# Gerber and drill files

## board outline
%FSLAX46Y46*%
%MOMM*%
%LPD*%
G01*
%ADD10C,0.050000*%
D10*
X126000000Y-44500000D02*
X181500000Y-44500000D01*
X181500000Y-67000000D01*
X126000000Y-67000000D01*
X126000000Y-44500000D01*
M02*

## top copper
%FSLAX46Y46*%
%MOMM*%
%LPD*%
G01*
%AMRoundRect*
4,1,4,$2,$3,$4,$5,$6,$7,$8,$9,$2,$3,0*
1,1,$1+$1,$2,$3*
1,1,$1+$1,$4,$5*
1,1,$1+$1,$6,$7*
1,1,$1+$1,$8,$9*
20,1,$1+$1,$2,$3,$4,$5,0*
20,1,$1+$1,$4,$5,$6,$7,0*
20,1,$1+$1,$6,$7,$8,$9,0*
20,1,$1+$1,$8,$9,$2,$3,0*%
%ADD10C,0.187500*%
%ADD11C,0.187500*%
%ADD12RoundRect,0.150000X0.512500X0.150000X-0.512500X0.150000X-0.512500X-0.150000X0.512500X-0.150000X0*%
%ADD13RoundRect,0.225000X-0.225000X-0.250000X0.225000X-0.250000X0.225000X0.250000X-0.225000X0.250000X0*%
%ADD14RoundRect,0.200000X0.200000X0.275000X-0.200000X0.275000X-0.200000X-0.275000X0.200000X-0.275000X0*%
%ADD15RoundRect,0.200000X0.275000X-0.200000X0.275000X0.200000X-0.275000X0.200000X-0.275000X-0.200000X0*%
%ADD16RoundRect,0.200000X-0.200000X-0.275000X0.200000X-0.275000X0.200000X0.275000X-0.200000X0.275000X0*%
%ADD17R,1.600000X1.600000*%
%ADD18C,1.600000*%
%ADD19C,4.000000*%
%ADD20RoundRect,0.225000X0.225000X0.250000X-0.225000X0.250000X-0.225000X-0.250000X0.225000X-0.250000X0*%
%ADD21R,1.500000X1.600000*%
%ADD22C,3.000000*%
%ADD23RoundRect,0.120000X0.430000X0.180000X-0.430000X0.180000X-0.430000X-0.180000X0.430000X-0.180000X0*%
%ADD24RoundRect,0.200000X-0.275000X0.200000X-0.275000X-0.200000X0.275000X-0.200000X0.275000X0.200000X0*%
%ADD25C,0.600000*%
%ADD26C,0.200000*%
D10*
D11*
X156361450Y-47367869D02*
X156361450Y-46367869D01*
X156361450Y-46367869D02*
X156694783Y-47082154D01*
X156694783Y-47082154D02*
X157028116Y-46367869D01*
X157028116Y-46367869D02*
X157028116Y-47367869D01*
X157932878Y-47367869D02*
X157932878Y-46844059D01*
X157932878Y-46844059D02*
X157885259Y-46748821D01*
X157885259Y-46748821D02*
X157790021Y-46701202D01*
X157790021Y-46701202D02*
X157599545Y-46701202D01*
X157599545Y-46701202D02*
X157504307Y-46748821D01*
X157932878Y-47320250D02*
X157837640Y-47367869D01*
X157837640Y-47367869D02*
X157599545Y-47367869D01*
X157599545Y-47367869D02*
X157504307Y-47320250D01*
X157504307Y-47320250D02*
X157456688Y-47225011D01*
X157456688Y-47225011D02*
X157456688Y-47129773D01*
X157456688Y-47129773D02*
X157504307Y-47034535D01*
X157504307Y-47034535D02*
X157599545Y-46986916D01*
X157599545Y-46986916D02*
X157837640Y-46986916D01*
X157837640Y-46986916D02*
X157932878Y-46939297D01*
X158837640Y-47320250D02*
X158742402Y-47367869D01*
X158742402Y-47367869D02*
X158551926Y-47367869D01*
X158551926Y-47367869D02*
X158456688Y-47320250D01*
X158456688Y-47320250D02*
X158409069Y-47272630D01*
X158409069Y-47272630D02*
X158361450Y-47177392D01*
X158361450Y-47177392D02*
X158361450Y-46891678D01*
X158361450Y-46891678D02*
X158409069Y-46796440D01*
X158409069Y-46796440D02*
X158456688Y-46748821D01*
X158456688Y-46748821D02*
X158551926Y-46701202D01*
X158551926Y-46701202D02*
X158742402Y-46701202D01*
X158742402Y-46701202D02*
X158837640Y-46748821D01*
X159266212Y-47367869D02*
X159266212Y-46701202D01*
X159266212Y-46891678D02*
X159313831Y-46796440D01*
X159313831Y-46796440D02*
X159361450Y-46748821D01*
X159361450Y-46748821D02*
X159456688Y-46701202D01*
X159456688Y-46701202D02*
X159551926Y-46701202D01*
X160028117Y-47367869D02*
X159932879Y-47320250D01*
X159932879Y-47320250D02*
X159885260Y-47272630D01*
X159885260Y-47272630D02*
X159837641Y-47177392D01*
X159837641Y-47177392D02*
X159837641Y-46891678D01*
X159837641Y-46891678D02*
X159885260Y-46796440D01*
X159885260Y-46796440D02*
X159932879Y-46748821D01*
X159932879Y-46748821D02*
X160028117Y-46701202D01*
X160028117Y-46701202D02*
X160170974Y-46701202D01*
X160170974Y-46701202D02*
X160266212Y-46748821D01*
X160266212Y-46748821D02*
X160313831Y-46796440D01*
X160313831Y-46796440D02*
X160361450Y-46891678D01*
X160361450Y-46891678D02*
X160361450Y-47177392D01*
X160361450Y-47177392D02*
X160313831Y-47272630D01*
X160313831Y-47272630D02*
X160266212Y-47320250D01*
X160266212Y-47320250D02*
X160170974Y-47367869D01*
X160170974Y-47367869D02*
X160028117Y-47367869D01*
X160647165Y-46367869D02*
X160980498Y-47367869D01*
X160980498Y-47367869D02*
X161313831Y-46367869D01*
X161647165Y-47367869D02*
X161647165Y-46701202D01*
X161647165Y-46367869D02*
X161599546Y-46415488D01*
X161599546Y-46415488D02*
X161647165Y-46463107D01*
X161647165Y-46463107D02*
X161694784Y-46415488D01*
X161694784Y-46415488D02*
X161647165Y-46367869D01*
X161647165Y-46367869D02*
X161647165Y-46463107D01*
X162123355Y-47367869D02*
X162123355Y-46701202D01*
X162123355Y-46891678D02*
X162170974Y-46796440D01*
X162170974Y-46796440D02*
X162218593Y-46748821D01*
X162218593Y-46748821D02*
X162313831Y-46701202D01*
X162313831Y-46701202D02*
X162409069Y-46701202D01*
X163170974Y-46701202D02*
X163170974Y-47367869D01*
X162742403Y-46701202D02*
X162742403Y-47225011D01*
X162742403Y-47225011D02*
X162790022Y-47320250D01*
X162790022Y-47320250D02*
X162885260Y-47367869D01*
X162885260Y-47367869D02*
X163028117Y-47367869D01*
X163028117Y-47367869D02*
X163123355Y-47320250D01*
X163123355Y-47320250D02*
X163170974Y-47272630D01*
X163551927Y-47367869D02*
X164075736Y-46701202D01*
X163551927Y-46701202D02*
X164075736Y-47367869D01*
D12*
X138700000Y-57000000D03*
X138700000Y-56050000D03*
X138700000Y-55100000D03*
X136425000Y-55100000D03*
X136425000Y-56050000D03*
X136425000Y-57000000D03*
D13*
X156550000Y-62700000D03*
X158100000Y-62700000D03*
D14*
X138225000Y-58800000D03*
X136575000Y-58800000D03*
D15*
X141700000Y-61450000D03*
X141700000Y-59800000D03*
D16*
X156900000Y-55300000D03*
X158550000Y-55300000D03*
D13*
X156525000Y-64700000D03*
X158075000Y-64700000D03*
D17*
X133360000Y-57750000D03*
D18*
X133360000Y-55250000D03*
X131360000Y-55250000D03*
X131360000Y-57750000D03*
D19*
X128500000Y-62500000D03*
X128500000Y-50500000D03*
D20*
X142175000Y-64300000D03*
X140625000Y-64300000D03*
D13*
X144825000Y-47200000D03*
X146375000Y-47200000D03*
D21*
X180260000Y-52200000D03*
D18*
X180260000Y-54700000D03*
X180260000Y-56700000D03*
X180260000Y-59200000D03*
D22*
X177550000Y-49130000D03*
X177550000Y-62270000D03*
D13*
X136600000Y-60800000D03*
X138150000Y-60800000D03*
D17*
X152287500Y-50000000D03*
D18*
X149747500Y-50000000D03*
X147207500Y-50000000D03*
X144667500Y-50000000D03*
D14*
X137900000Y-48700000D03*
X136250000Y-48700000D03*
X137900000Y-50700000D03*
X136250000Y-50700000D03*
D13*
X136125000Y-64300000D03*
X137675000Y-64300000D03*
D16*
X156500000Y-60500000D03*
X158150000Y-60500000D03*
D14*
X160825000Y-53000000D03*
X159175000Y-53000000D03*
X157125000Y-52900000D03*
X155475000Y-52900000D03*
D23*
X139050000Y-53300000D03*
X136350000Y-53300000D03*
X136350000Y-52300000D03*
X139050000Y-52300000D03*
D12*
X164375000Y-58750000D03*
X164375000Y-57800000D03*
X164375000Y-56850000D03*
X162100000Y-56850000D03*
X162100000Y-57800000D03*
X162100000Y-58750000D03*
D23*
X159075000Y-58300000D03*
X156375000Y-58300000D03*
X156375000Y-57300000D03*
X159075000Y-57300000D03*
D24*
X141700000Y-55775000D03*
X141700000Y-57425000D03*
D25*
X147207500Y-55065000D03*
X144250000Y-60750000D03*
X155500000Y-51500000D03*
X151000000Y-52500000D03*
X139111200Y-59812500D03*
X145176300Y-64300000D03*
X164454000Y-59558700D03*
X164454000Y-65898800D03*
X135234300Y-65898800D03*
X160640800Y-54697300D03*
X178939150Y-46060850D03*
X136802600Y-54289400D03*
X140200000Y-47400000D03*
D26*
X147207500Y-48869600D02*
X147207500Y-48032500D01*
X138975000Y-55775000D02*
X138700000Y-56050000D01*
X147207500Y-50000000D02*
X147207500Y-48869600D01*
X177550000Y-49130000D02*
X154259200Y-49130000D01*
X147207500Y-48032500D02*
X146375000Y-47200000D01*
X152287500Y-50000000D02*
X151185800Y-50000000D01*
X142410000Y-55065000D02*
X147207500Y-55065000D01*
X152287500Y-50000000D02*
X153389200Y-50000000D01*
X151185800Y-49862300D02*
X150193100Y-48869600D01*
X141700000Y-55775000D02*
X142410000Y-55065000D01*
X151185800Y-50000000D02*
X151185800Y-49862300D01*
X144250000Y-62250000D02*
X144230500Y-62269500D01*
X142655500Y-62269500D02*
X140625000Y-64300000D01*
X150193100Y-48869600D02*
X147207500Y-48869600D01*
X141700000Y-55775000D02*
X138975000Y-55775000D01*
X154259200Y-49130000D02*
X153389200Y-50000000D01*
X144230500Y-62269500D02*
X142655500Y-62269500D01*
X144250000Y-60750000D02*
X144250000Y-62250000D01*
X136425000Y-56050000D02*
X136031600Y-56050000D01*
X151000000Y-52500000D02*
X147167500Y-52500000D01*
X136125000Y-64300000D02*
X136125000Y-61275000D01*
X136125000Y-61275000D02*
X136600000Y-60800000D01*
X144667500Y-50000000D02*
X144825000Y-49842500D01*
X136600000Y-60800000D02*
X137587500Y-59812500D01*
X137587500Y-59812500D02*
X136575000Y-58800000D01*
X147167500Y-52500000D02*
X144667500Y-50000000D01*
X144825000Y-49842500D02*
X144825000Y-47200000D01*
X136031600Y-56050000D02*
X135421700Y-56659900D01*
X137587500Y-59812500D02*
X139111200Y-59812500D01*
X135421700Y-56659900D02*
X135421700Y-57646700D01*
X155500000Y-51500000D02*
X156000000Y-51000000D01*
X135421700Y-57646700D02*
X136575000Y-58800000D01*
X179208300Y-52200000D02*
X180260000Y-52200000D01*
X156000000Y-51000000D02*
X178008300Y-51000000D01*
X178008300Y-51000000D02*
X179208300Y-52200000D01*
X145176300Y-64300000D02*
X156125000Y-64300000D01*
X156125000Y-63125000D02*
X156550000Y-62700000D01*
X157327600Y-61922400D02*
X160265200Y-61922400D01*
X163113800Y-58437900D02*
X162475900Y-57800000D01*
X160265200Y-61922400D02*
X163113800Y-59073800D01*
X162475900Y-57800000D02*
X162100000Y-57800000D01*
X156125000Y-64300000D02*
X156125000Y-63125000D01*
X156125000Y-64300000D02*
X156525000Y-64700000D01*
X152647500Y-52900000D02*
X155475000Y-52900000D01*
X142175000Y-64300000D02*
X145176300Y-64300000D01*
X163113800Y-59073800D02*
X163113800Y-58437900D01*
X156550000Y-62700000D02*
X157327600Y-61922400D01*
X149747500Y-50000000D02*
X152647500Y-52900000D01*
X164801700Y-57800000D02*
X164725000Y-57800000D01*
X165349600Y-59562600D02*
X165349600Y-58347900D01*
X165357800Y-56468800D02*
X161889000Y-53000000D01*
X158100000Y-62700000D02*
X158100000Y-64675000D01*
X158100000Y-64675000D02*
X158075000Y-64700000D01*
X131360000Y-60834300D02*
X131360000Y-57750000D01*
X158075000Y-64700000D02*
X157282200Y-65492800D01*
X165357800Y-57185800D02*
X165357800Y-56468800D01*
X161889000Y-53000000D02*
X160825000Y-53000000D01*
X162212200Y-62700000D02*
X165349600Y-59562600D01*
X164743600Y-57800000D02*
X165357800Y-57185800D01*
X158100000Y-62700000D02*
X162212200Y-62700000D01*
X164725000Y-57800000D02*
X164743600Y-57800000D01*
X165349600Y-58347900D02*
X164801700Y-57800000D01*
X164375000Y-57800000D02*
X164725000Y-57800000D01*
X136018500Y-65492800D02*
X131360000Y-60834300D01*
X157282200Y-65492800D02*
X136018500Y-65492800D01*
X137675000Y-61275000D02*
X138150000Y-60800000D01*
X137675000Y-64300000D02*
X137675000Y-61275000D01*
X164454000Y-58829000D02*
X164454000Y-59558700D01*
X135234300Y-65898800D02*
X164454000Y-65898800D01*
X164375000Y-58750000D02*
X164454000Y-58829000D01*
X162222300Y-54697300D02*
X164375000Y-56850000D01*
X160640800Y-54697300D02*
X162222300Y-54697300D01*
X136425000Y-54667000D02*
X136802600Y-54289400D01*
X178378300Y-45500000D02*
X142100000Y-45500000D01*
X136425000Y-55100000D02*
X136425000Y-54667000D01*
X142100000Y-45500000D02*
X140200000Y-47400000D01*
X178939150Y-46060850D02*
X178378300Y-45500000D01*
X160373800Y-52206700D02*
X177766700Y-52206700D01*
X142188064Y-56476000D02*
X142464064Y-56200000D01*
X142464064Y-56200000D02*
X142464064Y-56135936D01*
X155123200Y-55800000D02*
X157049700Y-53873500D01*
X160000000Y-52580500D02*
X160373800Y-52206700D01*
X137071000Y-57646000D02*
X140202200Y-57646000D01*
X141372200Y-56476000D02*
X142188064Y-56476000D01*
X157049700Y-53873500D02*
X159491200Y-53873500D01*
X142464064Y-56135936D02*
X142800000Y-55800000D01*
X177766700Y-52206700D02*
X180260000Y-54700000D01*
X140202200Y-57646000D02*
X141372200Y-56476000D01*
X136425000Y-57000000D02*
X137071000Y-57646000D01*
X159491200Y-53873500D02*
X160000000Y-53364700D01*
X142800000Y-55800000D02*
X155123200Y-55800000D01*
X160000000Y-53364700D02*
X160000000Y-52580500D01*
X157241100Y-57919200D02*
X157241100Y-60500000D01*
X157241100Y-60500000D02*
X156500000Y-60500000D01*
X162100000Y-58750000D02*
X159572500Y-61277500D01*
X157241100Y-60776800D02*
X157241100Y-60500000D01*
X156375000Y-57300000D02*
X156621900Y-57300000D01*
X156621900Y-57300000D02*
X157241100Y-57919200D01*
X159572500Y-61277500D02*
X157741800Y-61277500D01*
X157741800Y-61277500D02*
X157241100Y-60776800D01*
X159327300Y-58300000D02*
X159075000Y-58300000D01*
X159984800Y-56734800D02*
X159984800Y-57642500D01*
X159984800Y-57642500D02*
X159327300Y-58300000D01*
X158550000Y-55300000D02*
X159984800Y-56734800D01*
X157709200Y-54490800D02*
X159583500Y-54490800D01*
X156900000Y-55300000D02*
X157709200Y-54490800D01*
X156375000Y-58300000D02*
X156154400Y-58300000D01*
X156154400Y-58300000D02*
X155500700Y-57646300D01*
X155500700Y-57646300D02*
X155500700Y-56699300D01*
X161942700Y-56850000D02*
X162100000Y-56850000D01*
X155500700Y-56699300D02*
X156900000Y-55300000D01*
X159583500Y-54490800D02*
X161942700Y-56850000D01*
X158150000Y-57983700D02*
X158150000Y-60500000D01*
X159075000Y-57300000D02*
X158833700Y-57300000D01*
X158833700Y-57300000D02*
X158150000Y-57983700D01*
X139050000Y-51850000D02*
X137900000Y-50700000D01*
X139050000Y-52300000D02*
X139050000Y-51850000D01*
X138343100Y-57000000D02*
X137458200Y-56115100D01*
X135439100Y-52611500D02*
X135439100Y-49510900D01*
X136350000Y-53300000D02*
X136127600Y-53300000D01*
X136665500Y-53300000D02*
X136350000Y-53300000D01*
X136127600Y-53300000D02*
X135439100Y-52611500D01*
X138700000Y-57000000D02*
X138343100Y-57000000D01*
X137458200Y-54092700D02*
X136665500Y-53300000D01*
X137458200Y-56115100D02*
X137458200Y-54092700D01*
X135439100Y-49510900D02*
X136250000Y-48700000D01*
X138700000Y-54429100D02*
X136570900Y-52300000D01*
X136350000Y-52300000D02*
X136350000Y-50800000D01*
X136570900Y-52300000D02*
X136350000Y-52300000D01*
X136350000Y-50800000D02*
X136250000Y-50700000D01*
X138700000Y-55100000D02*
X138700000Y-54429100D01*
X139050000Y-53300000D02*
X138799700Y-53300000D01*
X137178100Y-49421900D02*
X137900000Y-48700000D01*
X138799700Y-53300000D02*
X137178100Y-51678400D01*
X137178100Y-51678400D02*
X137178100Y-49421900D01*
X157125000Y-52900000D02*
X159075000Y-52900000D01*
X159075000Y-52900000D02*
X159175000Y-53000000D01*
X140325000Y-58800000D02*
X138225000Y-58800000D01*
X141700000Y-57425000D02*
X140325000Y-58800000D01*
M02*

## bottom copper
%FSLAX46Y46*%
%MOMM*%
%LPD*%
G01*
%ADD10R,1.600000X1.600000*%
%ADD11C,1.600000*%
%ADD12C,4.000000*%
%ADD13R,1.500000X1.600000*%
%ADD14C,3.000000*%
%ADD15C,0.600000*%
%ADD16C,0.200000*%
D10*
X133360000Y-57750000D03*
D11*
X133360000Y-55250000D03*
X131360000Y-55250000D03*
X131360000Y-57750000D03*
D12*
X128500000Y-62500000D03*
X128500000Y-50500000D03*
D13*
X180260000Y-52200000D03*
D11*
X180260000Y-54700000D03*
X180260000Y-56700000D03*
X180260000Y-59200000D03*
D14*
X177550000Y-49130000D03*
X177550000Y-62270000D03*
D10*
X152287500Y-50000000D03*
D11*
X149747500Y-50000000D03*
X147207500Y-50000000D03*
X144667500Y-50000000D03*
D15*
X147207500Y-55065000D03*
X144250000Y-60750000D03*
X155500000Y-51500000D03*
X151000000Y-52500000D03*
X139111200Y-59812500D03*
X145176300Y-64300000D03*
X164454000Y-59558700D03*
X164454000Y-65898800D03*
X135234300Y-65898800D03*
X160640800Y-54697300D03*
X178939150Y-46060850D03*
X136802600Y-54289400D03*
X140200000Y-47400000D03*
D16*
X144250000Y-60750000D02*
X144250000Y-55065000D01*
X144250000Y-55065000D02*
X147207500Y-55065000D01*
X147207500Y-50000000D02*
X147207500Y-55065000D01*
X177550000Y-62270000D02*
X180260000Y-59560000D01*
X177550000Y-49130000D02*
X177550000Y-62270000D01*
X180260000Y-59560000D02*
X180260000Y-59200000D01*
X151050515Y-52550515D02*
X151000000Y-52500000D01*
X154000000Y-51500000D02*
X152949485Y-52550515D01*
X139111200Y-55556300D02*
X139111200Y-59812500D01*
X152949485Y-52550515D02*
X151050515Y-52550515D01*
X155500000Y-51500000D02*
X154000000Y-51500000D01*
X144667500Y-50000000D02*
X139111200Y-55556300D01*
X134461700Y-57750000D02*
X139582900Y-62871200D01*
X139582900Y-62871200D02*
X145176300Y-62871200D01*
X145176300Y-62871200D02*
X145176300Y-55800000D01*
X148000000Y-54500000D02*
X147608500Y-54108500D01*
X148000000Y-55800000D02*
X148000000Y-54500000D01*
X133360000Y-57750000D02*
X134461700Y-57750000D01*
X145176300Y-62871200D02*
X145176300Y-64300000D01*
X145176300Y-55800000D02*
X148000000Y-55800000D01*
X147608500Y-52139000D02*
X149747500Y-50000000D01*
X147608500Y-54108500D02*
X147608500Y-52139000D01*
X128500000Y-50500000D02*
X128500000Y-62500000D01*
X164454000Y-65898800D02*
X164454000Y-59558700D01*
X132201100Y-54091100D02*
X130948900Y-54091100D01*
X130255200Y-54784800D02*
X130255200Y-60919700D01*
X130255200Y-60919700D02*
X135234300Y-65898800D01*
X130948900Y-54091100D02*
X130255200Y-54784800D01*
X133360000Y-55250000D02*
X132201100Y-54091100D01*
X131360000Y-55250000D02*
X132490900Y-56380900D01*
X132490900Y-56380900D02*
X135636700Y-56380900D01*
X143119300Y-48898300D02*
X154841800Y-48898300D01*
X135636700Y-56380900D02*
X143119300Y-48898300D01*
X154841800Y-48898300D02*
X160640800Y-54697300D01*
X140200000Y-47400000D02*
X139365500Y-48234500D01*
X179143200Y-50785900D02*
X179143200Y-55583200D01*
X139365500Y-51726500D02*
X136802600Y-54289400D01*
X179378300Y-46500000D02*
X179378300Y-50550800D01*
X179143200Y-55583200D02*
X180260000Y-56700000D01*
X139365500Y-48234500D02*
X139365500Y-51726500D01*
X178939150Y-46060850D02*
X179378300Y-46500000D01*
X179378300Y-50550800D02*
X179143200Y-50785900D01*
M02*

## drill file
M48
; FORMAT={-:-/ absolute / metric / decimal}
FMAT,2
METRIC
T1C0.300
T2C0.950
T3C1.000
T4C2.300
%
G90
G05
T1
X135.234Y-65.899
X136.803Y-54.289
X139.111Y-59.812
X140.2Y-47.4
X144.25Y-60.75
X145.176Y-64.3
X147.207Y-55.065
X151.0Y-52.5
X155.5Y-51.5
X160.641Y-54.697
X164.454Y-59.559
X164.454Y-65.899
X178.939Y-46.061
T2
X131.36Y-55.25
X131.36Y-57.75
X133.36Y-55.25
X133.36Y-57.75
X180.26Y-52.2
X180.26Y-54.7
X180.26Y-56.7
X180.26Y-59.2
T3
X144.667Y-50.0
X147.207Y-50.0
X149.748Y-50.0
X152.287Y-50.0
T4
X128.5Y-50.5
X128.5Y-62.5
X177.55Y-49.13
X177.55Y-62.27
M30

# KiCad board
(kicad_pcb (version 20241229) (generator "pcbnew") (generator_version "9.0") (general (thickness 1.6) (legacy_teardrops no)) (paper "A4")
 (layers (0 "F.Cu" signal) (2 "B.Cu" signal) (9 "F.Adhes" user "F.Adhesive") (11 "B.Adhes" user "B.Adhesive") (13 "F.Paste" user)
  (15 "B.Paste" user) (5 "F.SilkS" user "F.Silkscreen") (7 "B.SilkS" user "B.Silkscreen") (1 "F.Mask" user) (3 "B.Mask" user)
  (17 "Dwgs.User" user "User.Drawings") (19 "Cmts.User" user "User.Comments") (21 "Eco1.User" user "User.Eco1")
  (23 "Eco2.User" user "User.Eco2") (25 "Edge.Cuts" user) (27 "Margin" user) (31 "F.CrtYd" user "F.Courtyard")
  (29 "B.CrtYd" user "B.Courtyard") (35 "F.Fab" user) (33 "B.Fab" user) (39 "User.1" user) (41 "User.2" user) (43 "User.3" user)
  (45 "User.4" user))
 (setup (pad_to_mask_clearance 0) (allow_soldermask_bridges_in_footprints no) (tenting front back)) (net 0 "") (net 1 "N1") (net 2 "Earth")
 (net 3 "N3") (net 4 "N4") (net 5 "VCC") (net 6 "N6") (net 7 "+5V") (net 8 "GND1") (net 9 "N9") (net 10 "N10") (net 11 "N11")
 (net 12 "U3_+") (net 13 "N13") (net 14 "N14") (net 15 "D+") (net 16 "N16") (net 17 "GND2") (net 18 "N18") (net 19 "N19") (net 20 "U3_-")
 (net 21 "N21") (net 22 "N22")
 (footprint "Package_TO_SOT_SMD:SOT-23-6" (layer "F.Cu") (at 137.5625 56.05 180)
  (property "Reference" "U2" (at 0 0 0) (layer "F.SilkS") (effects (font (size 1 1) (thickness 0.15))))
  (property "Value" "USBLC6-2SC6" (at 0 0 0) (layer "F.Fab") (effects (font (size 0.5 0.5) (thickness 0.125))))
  (pad "1" smd roundrect (at -1.1375 -0.95 180) (size 1.325 0.6) (layers "F.Cu" "F.Mask" "F.Paste") (roundrect_rratio 0.25) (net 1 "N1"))
  (pad "2" smd roundrect (at -1.1375 0 180) (size 1.325 0.6) (layers "F.Cu" "F.Mask" "F.Paste") (roundrect_rratio 0.25) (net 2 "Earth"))
  (pad "3" smd roundrect (at -1.1375 0.95 180) (size 1.325 0.6) (layers "F.Cu" "F.Mask" "F.Paste") (roundrect_rratio 0.25) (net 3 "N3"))
  (pad "4" smd roundrect (at 1.1375 0.95 180) (size 1.325 0.6) (layers "F.Cu" "F.Mask" "F.Paste") (roundrect_rratio 0.25) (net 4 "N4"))
  (pad "5" smd roundrect (at 1.1375 0 180) (size 1.325 0.6) (layers "F.Cu" "F.Mask" "F.Paste") (roundrect_rratio 0.25) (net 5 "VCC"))
  (pad "6" smd roundrect (at 1.1375 -0.95 180) (size 1.325 0.6) (layers "F.Cu" "F.Mask" "F.Paste") (roundrect_rratio 0.25) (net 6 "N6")))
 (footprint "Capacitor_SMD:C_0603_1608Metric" (layer "F.Cu") (at 157.325 62.7)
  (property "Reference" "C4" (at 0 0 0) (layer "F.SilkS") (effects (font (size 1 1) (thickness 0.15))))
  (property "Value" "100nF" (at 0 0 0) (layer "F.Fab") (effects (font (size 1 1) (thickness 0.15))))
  (pad "1" smd roundrect (at -0.775 0) (size 0.9 0.95) (layers "F.Cu" "F.Mask" "F.Paste") (roundrect_rratio 0.25) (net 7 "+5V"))
  (pad "2" smd roundrect (at 0.775 0) (size 0.9 0.95) (layers "F.Cu" "F.Mask" "F.Paste") (roundrect_rratio 0.25) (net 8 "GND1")))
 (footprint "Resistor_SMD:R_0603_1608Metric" (layer "F.Cu") (at 137.4 58.8 180)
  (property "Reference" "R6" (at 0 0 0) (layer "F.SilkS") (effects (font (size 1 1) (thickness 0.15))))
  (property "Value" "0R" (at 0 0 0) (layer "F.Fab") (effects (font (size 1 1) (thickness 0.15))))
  (pad "1" smd roundrect (at -0.825 0 180) (size 0.8 0.95) (layers "F.Cu" "F.Mask" "F.Paste") (roundrect_rratio 0.25) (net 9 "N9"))
  (pad "2" smd roundrect (at 0.825 0 180) (size 0.8 0.95) (layers "F.Cu" "F.Mask" "F.Paste") (roundrect_rratio 0.25) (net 5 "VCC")))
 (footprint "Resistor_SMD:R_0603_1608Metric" (layer "F.Cu") (at 141.7 60.625 90)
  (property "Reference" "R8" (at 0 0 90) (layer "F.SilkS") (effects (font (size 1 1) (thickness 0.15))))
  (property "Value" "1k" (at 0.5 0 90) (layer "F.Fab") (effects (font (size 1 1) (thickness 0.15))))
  (pad "1" smd roundrect (at -0.825 0 90) (size 0.8 0.95) (layers "F.Cu" "F.Mask" "F.Paste") (roundrect_rratio 0.25) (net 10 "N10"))
  (pad "2" smd roundrect (at 0.825 0 90) (size 0.8 0.95) (layers "F.Cu" "F.Mask" "F.Paste") (roundrect_rratio 0.25) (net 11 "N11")))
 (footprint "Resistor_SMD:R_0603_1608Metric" (layer "F.Cu") (at 157.725 55.3)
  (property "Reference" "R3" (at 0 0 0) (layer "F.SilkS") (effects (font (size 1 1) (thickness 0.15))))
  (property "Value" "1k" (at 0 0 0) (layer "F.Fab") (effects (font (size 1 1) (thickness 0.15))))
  (pad "1" smd roundrect (at -0.825 0) (size 0.8 0.95) (layers "F.Cu" "F.Mask" "F.Paste") (roundrect_rratio 0.25) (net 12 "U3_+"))
  (pad "2" smd roundrect (at 0.825 0) (size 0.8 0.95) (layers "F.Cu" "F.Mask" "F.Paste") (roundrect_rratio 0.25) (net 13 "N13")))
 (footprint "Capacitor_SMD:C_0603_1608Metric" (layer "F.Cu") (at 157.3 64.7)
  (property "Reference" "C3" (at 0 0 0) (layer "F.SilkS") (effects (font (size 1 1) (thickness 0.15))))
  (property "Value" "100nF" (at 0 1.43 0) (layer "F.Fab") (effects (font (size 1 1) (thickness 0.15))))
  (pad "1" smd roundrect (at -0.775 0) (size 0.9 0.95) (layers "F.Cu" "F.Mask" "F.Paste") (roundrect_rratio 0.25) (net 7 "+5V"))
  (pad "2" smd roundrect (at 0.775 0) (size 0.9 0.95) (layers "F.Cu" "F.Mask" "F.Paste") (roundrect_rratio 0.25) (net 8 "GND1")))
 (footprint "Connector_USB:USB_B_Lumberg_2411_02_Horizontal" (layer "F.Cu") (at 133.36 57.75 180)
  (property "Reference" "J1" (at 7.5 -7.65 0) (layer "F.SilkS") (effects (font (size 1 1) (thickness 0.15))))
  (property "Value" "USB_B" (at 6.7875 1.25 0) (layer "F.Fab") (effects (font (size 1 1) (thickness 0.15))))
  (pad "1" thru_hole rect (at 0 0 270) (size 1.6 1.6) (drill 0.95) (layers "*.Cu" "*.Mask") (remove_unused_layers no) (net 7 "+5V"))
  (pad "2" thru_hole circle (at 0 2.5 270) (size 1.6 1.6) (drill 0.95) (layers "*.Cu" "*.Mask") (remove_unused_layers no) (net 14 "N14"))
  (pad "3" thru_hole circle (at 2 2.5 270) (size 1.6 1.6) (drill 0.95) (layers "*.Cu" "*.Mask") (remove_unused_layers no) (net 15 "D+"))
  (pad "4" thru_hole circle (at 2 0 270) (size 1.6 1.6) (drill 0.95) (layers "*.Cu" "*.Mask") (remove_unused_layers no) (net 8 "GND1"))
  (pad "5" thru_hole circle (at 4.86 -4.75 270) (size 4 4) (drill 2.3) (layers "*.Cu" "*.Mask") (remove_unused_layers no) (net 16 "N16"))
  (pad "5" thru_hole circle (at 4.86 7.25 270) (size 4 4) (drill 2.3) (layers "*.Cu" "*.Mask") (remove_unused_layers no) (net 16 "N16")))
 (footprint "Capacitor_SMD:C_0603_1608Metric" (layer "F.Cu") (at 141.4 64.3 180)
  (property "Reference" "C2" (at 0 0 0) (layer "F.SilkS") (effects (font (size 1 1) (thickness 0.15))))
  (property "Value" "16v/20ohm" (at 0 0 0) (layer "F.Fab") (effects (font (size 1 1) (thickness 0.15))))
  (pad "1" smd roundrect (at -0.775 0 180) (size 0.9 0.95) (layers "F.Cu" "F.Mask" "F.Paste") (roundrect_rratio 0.25) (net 7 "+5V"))
  (pad "2" smd roundrect (at 0.775 0 180) (size 0.9 0.95) (layers "F.Cu" "F.Mask" "F.Paste") (roundrect_rratio 0.25) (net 2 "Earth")))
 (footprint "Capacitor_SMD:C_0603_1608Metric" (layer "F.Cu") (at 145.6 47.2)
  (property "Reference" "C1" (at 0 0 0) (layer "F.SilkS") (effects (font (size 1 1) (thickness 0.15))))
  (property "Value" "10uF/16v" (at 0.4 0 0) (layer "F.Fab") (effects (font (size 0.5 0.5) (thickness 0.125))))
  (pad "1" smd roundrect (at -0.775 0) (size 0.9 0.95) (layers "F.Cu" "F.Mask" "F.Paste") (roundrect_rratio 0.25) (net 5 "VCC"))
  (pad "2" smd roundrect (at 0.775 0) (size 0.9 0.95) (layers "F.Cu" "F.Mask" "F.Paste") (roundrect_rratio 0.25) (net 2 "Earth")))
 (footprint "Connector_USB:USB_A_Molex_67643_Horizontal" (layer "F.Cu") (at 180.26 52.2 -90)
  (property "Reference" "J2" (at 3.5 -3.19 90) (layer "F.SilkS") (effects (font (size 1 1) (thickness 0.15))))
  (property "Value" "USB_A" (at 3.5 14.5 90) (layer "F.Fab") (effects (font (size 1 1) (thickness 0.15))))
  (pad "1" thru_hole rect (at 0 0 270) (size 1.6 1.5) (drill 0.95) (layers "*.Cu" "*.Mask") (remove_unused_layers no) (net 5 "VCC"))
  (pad "2" thru_hole circle (at 2.5 0 270) (size 1.6 1.6) (drill 0.95) (layers "*.Cu" "*.Mask") (remove_unused_layers no) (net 6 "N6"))
  (pad "3" thru_hole circle (at 4.5 0 270) (size 1.6 1.6) (drill 0.95) (layers "*.Cu" "*.Mask") (remove_unused_layers no) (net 4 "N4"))
  (pad "4" thru_hole circle (at 7 0 270) (size 1.6 1.6) (drill 0.95) (layers "*.Cu" "*.Mask") (remove_unused_layers no) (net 2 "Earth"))
  (pad "5" thru_hole circle (at -3.07 2.71 270) (size 3 3) (drill 2.3) (layers "*.Cu" "*.Mask") (remove_unused_layers no) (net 2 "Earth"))
  (pad "5" thru_hole circle (at 10.07 2.71 270) (size 3 3) (drill 2.3) (layers "*.Cu" "*.Mask") (remove_unused_layers no) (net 2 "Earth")))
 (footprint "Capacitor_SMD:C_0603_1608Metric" (layer "F.Cu") (at 137.375 60.8)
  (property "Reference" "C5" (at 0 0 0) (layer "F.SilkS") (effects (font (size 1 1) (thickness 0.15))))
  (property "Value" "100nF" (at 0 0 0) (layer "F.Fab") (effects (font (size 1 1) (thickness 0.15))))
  (pad "1" smd roundrect (at -0.775 0) (size 0.9 0.95) (layers "F.Cu" "F.Mask" "F.Paste") (roundrect_rratio 0.25) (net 5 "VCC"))
  (pad "2" smd roundrect (at 0.775 0) (size 0.9 0.95) (layers "F.Cu" "F.Mask" "F.Paste") (roundrect_rratio 0.25) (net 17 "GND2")))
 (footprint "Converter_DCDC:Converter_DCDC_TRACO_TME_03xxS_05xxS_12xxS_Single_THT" (layer "F.Cu") (at 152.2875 50 -90)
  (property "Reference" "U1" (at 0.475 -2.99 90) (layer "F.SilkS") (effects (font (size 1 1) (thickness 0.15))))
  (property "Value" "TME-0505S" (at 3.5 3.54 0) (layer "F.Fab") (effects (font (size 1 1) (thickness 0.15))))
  (pad "1" thru_hole rect (at 0 0 270) (size 1.6 1.6) (drill 1) (layers "*.Cu" "*.Mask") (remove_unused_layers no) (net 2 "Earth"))
  (pad "2" thru_hole circle (at 0 2.54 270) (size 1.6 1.6) (drill 1) (layers "*.Cu" "*.Mask") (remove_unused_layers no) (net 7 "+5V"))
  (pad "3" thru_hole circle (at 0 5.08 270) (size 1.6 1.6) (drill 1) (layers "*.Cu" "*.Mask") (remove_unused_layers no) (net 2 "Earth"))
  (pad "4" thru_hole circle (at 0 7.62 270) (size 1.6 1.6) (drill 1) (layers "*.Cu" "*.Mask") (remove_unused_layers no) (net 5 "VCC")))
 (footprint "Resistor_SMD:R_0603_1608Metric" (layer "F.Cu") (at 137.075 48.7 180)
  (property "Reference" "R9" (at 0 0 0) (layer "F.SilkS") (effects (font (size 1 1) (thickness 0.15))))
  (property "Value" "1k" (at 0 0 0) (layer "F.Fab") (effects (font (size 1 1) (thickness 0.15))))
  (pad "1" smd roundrect (at -0.825 0 180) (size 0.8 0.95) (layers "F.Cu" "F.Mask" "F.Paste") (roundrect_rratio 0.25) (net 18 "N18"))
  (pad "2" smd roundrect (at 0.825 0 180) (size 0.8 0.95) (layers "F.Cu" "F.Mask" "F.Paste") (roundrect_rratio 0.25) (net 1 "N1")))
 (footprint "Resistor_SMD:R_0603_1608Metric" (layer "F.Cu") (at 137.075 50.7 180)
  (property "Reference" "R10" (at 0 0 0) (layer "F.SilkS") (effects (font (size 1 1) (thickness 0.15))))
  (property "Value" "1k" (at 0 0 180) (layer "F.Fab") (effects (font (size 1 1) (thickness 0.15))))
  (pad "1" smd roundrect (at -0.825 0 180) (size 0.8 0.95) (layers "F.Cu" "F.Mask" "F.Paste") (roundrect_rratio 0.25) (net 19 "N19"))
  (pad "2" smd roundrect (at 0.825 0 180) (size 0.8 0.95) (layers "F.Cu" "F.Mask" "F.Paste") (roundrect_rratio 0.25) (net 3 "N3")))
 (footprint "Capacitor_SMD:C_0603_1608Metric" (layer "F.Cu") (at 136.9 64.3)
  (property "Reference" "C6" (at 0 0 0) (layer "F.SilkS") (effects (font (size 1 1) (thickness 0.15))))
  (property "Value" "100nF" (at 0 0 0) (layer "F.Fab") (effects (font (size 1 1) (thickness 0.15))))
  (pad "1" smd roundrect (at -0.775 0) (size 0.9 0.95) (layers "F.Cu" "F.Mask" "F.Paste") (roundrect_rratio 0.25) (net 5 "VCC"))
  (pad "2" smd roundrect (at 0.775 0) (size 0.9 0.95) (layers "F.Cu" "F.Mask" "F.Paste") (roundrect_rratio 0.25) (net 17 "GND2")))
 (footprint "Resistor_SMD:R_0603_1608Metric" (layer "F.Cu") (at 157.325 60.5)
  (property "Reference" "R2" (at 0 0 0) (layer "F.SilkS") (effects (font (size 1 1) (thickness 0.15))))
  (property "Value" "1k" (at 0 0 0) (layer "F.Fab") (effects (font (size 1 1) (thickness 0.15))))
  (pad "1" smd roundrect (at -0.825 0) (size 0.8 0.95) (layers "F.Cu" "F.Mask" "F.Paste") (roundrect_rratio 0.25) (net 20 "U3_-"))
  (pad "2" smd roundrect (at 0.825 0) (size 0.8 0.95) (layers "F.Cu" "F.Mask" "F.Paste") (roundrect_rratio 0.25) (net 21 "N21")))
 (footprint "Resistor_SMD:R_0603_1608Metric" (layer "F.Cu") (at 160 53 180)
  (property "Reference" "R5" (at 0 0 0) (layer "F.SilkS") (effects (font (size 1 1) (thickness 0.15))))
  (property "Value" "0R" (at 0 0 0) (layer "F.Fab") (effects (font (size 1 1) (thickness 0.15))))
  (pad "1" smd roundrect (at -0.825 0 180) (size 0.8 0.95) (layers "F.Cu" "F.Mask" "F.Paste") (roundrect_rratio 0.25) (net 8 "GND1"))
  (pad "2" smd roundrect (at 0.825 0 180) (size 0.8 0.95) (layers "F.Cu" "F.Mask" "F.Paste") (roundrect_rratio 0.25) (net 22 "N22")))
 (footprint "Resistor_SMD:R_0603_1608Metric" (layer "F.Cu") (at 156.3 52.9 180)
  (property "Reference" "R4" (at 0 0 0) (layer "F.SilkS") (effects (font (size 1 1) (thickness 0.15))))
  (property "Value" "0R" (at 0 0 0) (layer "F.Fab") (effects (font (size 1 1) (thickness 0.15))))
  (pad "1" smd roundrect (at -0.825 0 180) (size 0.8 0.95) (layers "F.Cu" "F.Mask" "F.Paste") (roundrect_rratio 0.25) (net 22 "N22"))
  (pad "2" smd roundrect (at 0.825 0 180) (size 0.8 0.95) (layers "F.Cu" "F.Mask" "F.Paste") (roundrect_rratio 0.25) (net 7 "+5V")))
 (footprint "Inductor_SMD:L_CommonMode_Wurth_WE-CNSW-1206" (layer "F.Cu") (at 137.7 52.8 180)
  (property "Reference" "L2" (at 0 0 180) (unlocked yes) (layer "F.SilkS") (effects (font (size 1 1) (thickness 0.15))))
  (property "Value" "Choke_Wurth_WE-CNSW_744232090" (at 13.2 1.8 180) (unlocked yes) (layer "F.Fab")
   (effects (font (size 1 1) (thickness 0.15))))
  (pad "1" smd roundrect (at -1.35 -0.5 180) (size 1.1 0.6) (layers "F.Cu" "F.Mask" "F.Paste") (roundrect_rratio 0.2) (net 18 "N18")
   (thermal_bridge_angle 45))
  (pad "2" smd roundrect (at 1.35 -0.5 180) (size 1.1 0.6) (layers "F.Cu" "F.Mask" "F.Paste") (roundrect_rratio 0.2) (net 1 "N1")
   (thermal_bridge_angle 45))
  (pad "3" smd roundrect (at 1.35 0.5 180) (size 1.1 0.6) (layers "F.Cu" "F.Mask" "F.Paste") (roundrect_rratio 0.2) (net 3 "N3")
   (thermal_bridge_angle 45))
  (pad "4" smd roundrect (at -1.35 0.5 180) (size 1.1 0.6) (layers "F.Cu" "F.Mask" "F.Paste") (roundrect_rratio 0.2) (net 19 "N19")
   (thermal_bridge_angle 45)))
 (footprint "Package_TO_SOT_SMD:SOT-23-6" (layer "F.Cu") (at 163.2375 57.8 180)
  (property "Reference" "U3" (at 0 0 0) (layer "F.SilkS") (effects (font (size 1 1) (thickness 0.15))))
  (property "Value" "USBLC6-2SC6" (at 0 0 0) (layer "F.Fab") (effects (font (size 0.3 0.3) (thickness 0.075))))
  (pad "1" smd roundrect (at -1.1375 -0.95 180) (size 1.325 0.6) (layers "F.Cu" "F.Mask" "F.Paste") (roundrect_rratio 0.25) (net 14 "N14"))
  (pad "2" smd roundrect (at -1.1375 0 180) (size 1.325 0.6) (layers "F.Cu" "F.Mask" "F.Paste") (roundrect_rratio 0.25) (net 8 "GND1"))
  (pad "3" smd roundrect (at -1.1375 0.95 180) (size 1.325 0.6) (layers "F.Cu" "F.Mask" "F.Paste") (roundrect_rratio 0.25) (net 15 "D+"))
  (pad "4" smd roundrect (at 1.1375 0.95 180) (size 1.325 0.6) (layers "F.Cu" "F.Mask" "F.Paste") (roundrect_rratio 0.25) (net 12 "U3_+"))
  (pad "5" smd roundrect (at 1.1375 0 180) (size 1.325 0.6) (layers "F.Cu" "F.Mask" "F.Paste") (roundrect_rratio 0.25) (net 7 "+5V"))
  (pad "6" smd roundrect (at 1.1375 -0.95 180) (size 1.325 0.6) (layers "F.Cu" "F.Mask" "F.Paste") (roundrect_rratio 0.25) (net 20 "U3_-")))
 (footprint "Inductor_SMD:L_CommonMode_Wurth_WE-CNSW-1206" (layer "F.Cu") (at 157.725 57.8 180)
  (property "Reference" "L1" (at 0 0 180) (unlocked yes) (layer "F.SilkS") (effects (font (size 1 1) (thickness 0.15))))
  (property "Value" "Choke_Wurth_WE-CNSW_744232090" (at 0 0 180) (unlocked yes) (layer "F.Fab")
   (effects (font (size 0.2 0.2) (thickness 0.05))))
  (pad "1" smd roundrect (at -1.35 -0.5 180) (size 1.1 0.6) (layers "F.Cu" "F.Mask" "F.Paste") (roundrect_rratio 0.2) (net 13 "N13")
   (thermal_bridge_angle 45))
  (pad "2" smd roundrect (at 1.35 -0.5 180) (size 1.1 0.6) (layers "F.Cu" "F.Mask" "F.Paste") (roundrect_rratio 0.2) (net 12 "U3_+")
   (thermal_bridge_angle 45))
  (pad "3" smd roundrect (at 1.35 0.5 180) (size 1.1 0.6) (layers "F.Cu" "F.Mask" "F.Paste") (roundrect_rratio 0.2) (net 20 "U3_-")
   (thermal_bridge_angle 45))
  (pad "4" smd roundrect (at -1.35 0.5 180) (size 1.1 0.6) (layers "F.Cu" "F.Mask" "F.Paste") (roundrect_rratio 0.2) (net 21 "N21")
   (thermal_bridge_angle 45)))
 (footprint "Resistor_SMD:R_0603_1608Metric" (layer "F.Cu") (at 141.7 56.6 -90)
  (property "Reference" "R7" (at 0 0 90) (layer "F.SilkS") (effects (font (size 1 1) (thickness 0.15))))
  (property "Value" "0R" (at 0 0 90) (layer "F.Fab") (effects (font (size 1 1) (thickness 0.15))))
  (pad "1" smd roundrect (at -0.825 0 270) (size 0.8 0.95) (layers "F.Cu" "F.Mask" "F.Paste") (roundrect_rratio 0.25) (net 2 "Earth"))
  (pad "2" smd roundrect (at 0.825 0 270) (size 0.8 0.95) (layers "F.Cu" "F.Mask" "F.Paste") (roundrect_rratio 0.25) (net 9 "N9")))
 (gr_rect (start 126 44.5) (end 181.5 67) (stroke (width 0.05) (type default)) (fill no) (layer "Edge.Cuts"))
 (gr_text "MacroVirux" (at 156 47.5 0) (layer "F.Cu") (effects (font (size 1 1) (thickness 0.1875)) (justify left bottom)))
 (segment (start 147.2075 48.8696) (end 147.2075 48.0325) (width 0.2) (layer "F.Cu") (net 2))
 (segment (start 138.975 55.775) (end 138.7 56.05) (width 0.2) (layer "F.Cu") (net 2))
 (segment (start 147.2075 50) (end 147.2075 48.8696) (width 0.2) (layer "F.Cu") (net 2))
 (segment (start 177.55 49.13) (end 154.2592 49.13) (width 0.2) (layer "F.Cu") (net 2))
 (segment (start 147.2075 48.0325) (end 146.375 47.2) (width 0.2) (layer "F.Cu") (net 2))
 (segment (start 152.2875 50) (end 151.1858 50) (width 0.2) (layer "F.Cu") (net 2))
 (segment (start 142.41 55.065) (end 147.2075 55.065) (width 0.2) (layer "F.Cu") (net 2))
 (segment (start 152.2875 50) (end 153.3892 50) (width 0.2) (layer "F.Cu") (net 2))
 (segment (start 151.1858 49.8623) (end 150.1931 48.8696) (width 0.2) (layer "F.Cu") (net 2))
 (segment (start 141.7 55.775) (end 142.41 55.065) (width 0.2) (layer "F.Cu") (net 2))
 (segment (start 151.1858 50) (end 151.1858 49.8623) (width 0.2) (layer "F.Cu") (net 2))
 (segment (start 144.25 62.25) (end 144.2305 62.2695) (width 0.2) (layer "F.Cu") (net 2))
 (segment (start 142.6555 62.2695) (end 140.625 64.3) (width 0.2) (layer "F.Cu") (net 2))
 (segment (start 150.1931 48.8696) (end 147.2075 48.8696) (width 0.2) (layer "F.Cu") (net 2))
 (segment (start 141.7 55.775) (end 138.975 55.775) (width 0.2) (layer "F.Cu") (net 2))
 (segment (start 154.2592 49.13) (end 153.3892 50) (width 0.2) (layer "F.Cu") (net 2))
 (segment (start 144.2305 62.2695) (end 142.6555 62.2695) (width 0.2) (layer "F.Cu") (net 2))
 (segment (start 144.25 60.75) (end 144.25 62.25) (width 0.2) (layer "F.Cu") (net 2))
 (via (at 147.2075 55.065) (size 0.6) (drill 0.3) (layers "F.Cu" "B.Cu") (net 2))
 (via (at 144.25 60.75) (size 0.6) (drill 0.3) (layers "F.Cu" "B.Cu") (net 2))
 (segment (start 144.25 60.75) (end 144.25 55.065) (width 0.2) (layer "B.Cu") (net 2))
 (segment (start 144.25 55.065) (end 147.2075 55.065) (width 0.2) (layer "B.Cu") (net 2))
 (segment (start 147.2075 50) (end 147.2075 55.065) (width 0.2) (layer "B.Cu") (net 2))
 (segment (start 177.55 62.27) (end 180.26 59.56) (width 0.2) (layer "B.Cu") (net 2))
 (segment (start 177.55 49.13) (end 177.55 62.27) (width 0.2) (layer "B.Cu") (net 2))
 (segment (start 180.26 59.56) (end 180.26 59.2) (width 0.2) (layer "B.Cu") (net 2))
 (segment (start 136.425 56.05) (end 136.0316 56.05) (width 0.2) (layer "F.Cu") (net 5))
 (segment (start 151 52.5) (end 147.1675 52.5) (width 0.2) (layer "F.Cu") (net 5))
 (segment (start 136.125 64.3) (end 136.125 61.275) (width 0.2) (layer "F.Cu") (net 5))
 (segment (start 136.125 61.275) (end 136.6 60.8) (width 0.2) (layer "F.Cu") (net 5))
 (segment (start 144.6675 50) (end 144.825 49.8425) (width 0.2) (layer "F.Cu") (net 5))
 (segment (start 136.6 60.8) (end 137.5875 59.8125) (width 0.2) (layer "F.Cu") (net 5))
 (segment (start 137.5875 59.8125) (end 136.575 58.8) (width 0.2) (layer "F.Cu") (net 5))
 (segment (start 147.1675 52.5) (end 144.6675 50) (width 0.2) (layer "F.Cu") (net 5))
 (segment (start 144.825 49.8425) (end 144.825 47.2) (width 0.2) (layer "F.Cu") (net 5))
 (segment (start 136.0316 56.05) (end 135.4217 56.6599) (width 0.2) (layer "F.Cu") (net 5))
 (segment (start 137.5875 59.8125) (end 139.1112 59.8125) (width 0.2) (layer "F.Cu") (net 5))
 (segment (start 135.4217 56.6599) (end 135.4217 57.6467) (width 0.2) (layer "F.Cu") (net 5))
 (segment (start 155.5 51.5) (end 156 51) (width 0.2) (layer "F.Cu") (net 5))
 (segment (start 135.4217 57.6467) (end 136.575 58.8) (width 0.2) (layer "F.Cu") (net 5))
 (segment (start 179.2083 52.2) (end 180.26 52.2) (width 0.2) (layer "F.Cu") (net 5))
 (segment (start 156 51) (end 178.0083 51) (width 0.2) (layer "F.Cu") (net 5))
 (segment (start 178.0083 51) (end 179.2083 52.2) (width 0.2) (layer "F.Cu") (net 5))
 (via (at 155.5 51.5) (size 0.6) (drill 0.3) (layers "F.Cu" "B.Cu") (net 5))
 (via (at 151 52.5) (size 0.6) (drill 0.3) (layers "F.Cu" "B.Cu") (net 5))
 (via (at 139.1112 59.8125) (size 0.6) (drill 0.3) (layers "F.Cu" "B.Cu") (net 5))
 (segment (start 151.050515 52.550515) (end 151 52.5) (width 0.2) (layer "B.Cu") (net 5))
 (segment (start 154 51.5) (end 152.949485 52.550515) (width 0.2) (layer "B.Cu") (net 5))
 (segment (start 139.1112 55.5563) (end 139.1112 59.8125) (width 0.2) (layer "B.Cu") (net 5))
 (segment (start 152.949485 52.550515) (end 151.050515 52.550515) (width 0.2) (layer "B.Cu") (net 5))
 (segment (start 155.5 51.5) (end 154 51.5) (width 0.2) (layer "B.Cu") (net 5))
 (segment (start 144.6675 50) (end 139.1112 55.5563) (width 0.2) (layer "B.Cu") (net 5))
 (segment (start 145.1763 64.3) (end 156.125 64.3) (width 0.2) (layer "F.Cu") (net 7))
 (segment (start 156.125 63.125) (end 156.55 62.7) (width 0.2) (layer "F.Cu") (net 7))
 (segment (start 157.3276 61.9224) (end 160.2652 61.9224) (width 0.2) (layer "F.Cu") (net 7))
 (segment (start 163.1138 58.4379) (end 162.4759 57.8) (width 0.2) (layer "F.Cu") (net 7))
 (segment (start 160.2652 61.9224) (end 163.1138 59.0738) (width 0.2) (layer "F.Cu") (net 7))
 (segment (start 162.4759 57.8) (end 162.1 57.8) (width 0.2) (layer "F.Cu") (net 7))
 (segment (start 156.125 64.3) (end 156.125 63.125) (width 0.2) (layer "F.Cu") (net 7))
 (segment (start 156.125 64.3) (end 156.525 64.7) (width 0.2) (layer "F.Cu") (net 7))
 (segment (start 152.6475 52.9) (end 155.475 52.9) (width 0.2) (layer "F.Cu") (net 7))
 (segment (start 142.175 64.3) (end 145.1763 64.3) (width 0.2) (layer "F.Cu") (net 7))
 (segment (start 163.1138 59.0738) (end 163.1138 58.4379) (width 0.2) (layer "F.Cu") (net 7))
 (segment (start 156.55 62.7) (end 157.3276 61.9224) (width 0.2) (layer "F.Cu") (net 7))
 (segment (start 149.7475 50) (end 152.6475 52.9) (width 0.2) (layer "F.Cu") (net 7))
 (via (at 145.1763 64.3) (size 0.6) (drill 0.3) (layers "F.Cu" "B.Cu") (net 7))
 (segment (start 134.4617 57.75) (end 139.5829 62.8712) (width 0.2) (layer "B.Cu") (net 7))
 (segment (start 139.5829 62.8712) (end 145.1763 62.8712) (width 0.2) (layer "B.Cu") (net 7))
 (segment (start 145.1763 62.8712) (end 145.1763 55.8) (width 0.2) (layer "B.Cu") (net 7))
 (segment (start 148 54.5) (end 147.6085 54.1085) (width 0.2) (layer "B.Cu") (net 7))
 (segment (start 148 55.8) (end 148 54.5) (width 0.2) (layer "B.Cu") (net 7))
 (segment (start 133.36 57.75) (end 134.4617 57.75) (width 0.2) (layer "B.Cu") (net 7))
 (segment (start 145.1763 62.8712) (end 145.1763 64.3) (width 0.2) (layer "B.Cu") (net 7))
 (segment (start 145.1763 55.8) (end 148 55.8) (width 0.2) (layer "B.Cu") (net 7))
 (segment (start 147.6085 52.139) (end 149.7475 50) (width 0.2) (layer "B.Cu") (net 7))
 (segment (start 147.6085 54.1085) (end 147.6085 52.139) (width 0.2) (layer "B.Cu") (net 7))
 (segment (start 164.8017 57.8) (end 164.725 57.8) (width 0.2) (layer "F.Cu") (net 8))
 (segment (start 165.3496 59.5626) (end 165.3496 58.3479) (width 0.2) (layer "F.Cu") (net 8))
 (segment (start 165.3578 56.4688) (end 161.889 53) (width 0.2) (layer "F.Cu") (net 8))
 (segment (start 158.1 62.7) (end 158.1 64.675) (width 0.2) (layer "F.Cu") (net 8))
 (segment (start 158.1 64.675) (end 158.075 64.7) (width 0.2) (layer "F.Cu") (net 8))
 (segment (start 131.36 60.8343) (end 131.36 57.75) (width 0.2) (layer "F.Cu") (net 8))
 (segment (start 158.075 64.7) (end 157.2822 65.4928) (width 0.2) (layer "F.Cu") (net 8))
 (segment (start 165.3578 57.1858) (end 165.3578 56.4688) (width 0.2) (layer "F.Cu") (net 8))
 (segment (start 161.889 53) (end 160.825 53) (width 0.2) (layer "F.Cu") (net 8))
 (segment (start 162.2122 62.7) (end 165.3496 59.5626) (width 0.2) (layer "F.Cu") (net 8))
 (segment (start 164.7436 57.8) (end 165.3578 57.1858) (width 0.2) (layer "F.Cu") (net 8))
 (segment (start 158.1 62.7) (end 162.2122 62.7) (width 0.2) (layer "F.Cu") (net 8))
 (segment (start 164.725 57.8) (end 164.7436 57.8) (width 0.2) (layer "F.Cu") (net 8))
 (segment (start 165.3496 58.3479) (end 164.8017 57.8) (width 0.2) (layer "F.Cu") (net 8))
 (segment (start 164.375 57.8) (end 164.725 57.8) (width 0.2) (layer "F.Cu") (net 8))
 (segment (start 136.0185 65.4928) (end 131.36 60.8343) (width 0.2) (layer "F.Cu") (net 8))
 (segment (start 157.2822 65.4928) (end 136.0185 65.4928) (width 0.2) (layer "F.Cu") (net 8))
 (segment (start 137.675 61.275) (end 138.15 60.8) (width 0.2) (layer "F.Cu") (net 17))
 (segment (start 137.675 64.3) (end 137.675 61.275) (width 0.2) (layer "F.Cu") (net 17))
 (segment (start 128.5 50.5) (end 128.5 62.5) (width 0.2) (layer "B.Cu") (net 16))
 (segment (start 164.454 58.829) (end 164.454 59.5587) (width 0.2) (layer "F.Cu") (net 14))
 (segment (start 135.2343 65.8988) (end 164.454 65.8988) (width 0.2) (layer "F.Cu") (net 14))
 (segment (start 164.375 58.75) (end 164.454 58.829) (width 0.2) (layer "F.Cu") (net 14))
 (via (at 164.454 59.5587) (size 0.6) (drill 0.3) (layers "F.Cu" "B.Cu") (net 14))
 (via (at 164.454 65.8988) (size 0.6) (drill 0.3) (layers "F.Cu" "B.Cu") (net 14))
 (via (at 135.2343 65.8988) (size 0.6) (drill 0.3) (layers "F.Cu" "B.Cu") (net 14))
 (segment (start 164.454 65.8988) (end 164.454 59.5587) (width 0.2) (layer "B.Cu") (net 14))
 (segment (start 132.2011 54.0911) (end 130.9489 54.0911) (width 0.2) (layer "B.Cu") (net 14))
 (segment (start 130.2552 54.7848) (end 130.2552 60.9197) (width 0.2) (layer "B.Cu") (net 14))
 (segment (start 130.2552 60.9197) (end 135.2343 65.8988) (width 0.2) (layer "B.Cu") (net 14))
 (segment (start 130.9489 54.0911) (end 130.2552 54.7848) (width 0.2) (layer "B.Cu") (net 14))
 (segment (start 133.36 55.25) (end 132.2011 54.0911) (width 0.2) (layer "B.Cu") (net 14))
 (segment (start 162.2223 54.6973) (end 164.375 56.85) (width 0.2) (layer "F.Cu") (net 15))
 (segment (start 160.6408 54.6973) (end 162.2223 54.6973) (width 0.2) (layer "F.Cu") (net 15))
 (via (at 160.6408 54.6973) (size 0.6) (drill 0.3) (layers "F.Cu" "B.Cu") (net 15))
 (segment (start 131.36 55.25) (end 132.4909 56.3809) (width 0.2) (layer "B.Cu") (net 15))
 (segment (start 132.4909 56.3809) (end 135.6367 56.3809) (width 0.2) (layer "B.Cu") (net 15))
 (segment (start 143.1193 48.8983) (end 154.8418 48.8983) (width 0.2) (layer "B.Cu") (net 15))
 (segment (start 135.6367 56.3809) (end 143.1193 48.8983) (width 0.2) (layer "B.Cu") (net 15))
 (segment (start 154.8418 48.8983) (end 160.6408 54.6973) (width 0.2) (layer "B.Cu") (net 15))
 (segment (start 136.425 54.667) (end 136.8026 54.2894) (width 0.2) (layer "F.Cu") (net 4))
 (segment (start 178.3783 45.5) (end 142.1 45.5) (width 0.2) (layer "F.Cu") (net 4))
 (segment (start 136.425 55.1) (end 136.425 54.667) (width 0.2) (layer "F.Cu") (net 4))
 (segment (start 142.1 45.5) (end 140.2 47.4) (width 0.2) (layer "F.Cu") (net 4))
 (segment (start 178.93915 46.06085) (end 178.3783 45.5) (width 0.2) (layer "F.Cu") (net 4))
 (via (at 178.93915 46.06085) (size 0.6) (drill 0.3) (layers "F.Cu" "B.Cu") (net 4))
 (via (at 136.8026 54.2894) (size 0.6) (drill 0.3) (layers "F.Cu" "B.Cu") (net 4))
 (via (at 140.2 47.4) (size 0.6) (drill 0.3) (layers "F.Cu" "B.Cu") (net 4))
 (segment (start 140.2 47.4) (end 139.3655 48.2345) (width 0.2) (layer "B.Cu") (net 4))
 (segment (start 179.1432 50.7859) (end 179.1432 55.5832) (width 0.2) (layer "B.Cu") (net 4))
 (segment (start 139.3655 51.7265) (end 136.8026 54.2894) (width 0.2) (layer "B.Cu") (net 4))
 (segment (start 179.3783 46.5) (end 179.3783 50.5508) (width 0.2) (layer "B.Cu") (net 4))
 (segment (start 179.1432 55.5832) (end 180.26 56.7) (width 0.2) (layer "B.Cu") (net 4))
 (segment (start 139.3655 48.2345) (end 139.3655 51.7265) (width 0.2) (layer "B.Cu") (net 4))
 (segment (start 178.93915 46.06085) (end 179.3783 46.5) (width 0.2) (layer "B.Cu") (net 4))
 (segment (start 179.3783 50.5508) (end 179.1432 50.7859) (width 0.2) (layer "B.Cu") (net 4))
 (segment (start 160.3738 52.2067) (end 177.7667 52.2067) (width 0.2) (layer "F.Cu") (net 6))
 (segment (start 142.188064 56.476) (end 142.464064 56.2) (width 0.2) (layer "F.Cu") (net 6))
 (segment (start 142.464064 56.2) (end 142.464064 56.135936) (width 0.2) (layer "F.Cu") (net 6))
 (segment (start 155.1232 55.8) (end 157.0497 53.8735) (width 0.2) (layer "F.Cu") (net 6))
 (segment (start 160 52.5805) (end 160.3738 52.2067) (width 0.2) (layer "F.Cu") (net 6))
 (segment (start 137.071 57.646) (end 140.2022 57.646) (width 0.2) (layer "F.Cu") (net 6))
 (segment (start 141.3722 56.476) (end 142.188064 56.476) (width 0.2) (layer "F.Cu") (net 6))
 (segment (start 157.0497 53.8735) (end 159.4912 53.8735) (width 0.2) (layer "F.Cu") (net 6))
 (segment (start 142.464064 56.135936) (end 142.8 55.8) (width 0.2) (layer "F.Cu") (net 6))
 (segment (start 177.7667 52.2067) (end 180.26 54.7) (width 0.2) (layer "F.Cu") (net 6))
 (segment (start 140.2022 57.646) (end 141.3722 56.476) (width 0.2) (layer "F.Cu") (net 6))
 (segment (start 136.425 57) (end 137.071 57.646) (width 0.2) (layer "F.Cu") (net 6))
 (segment (start 159.4912 53.8735) (end 160 53.3647) (width 0.2) (layer "F.Cu") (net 6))
 (segment (start 142.8 55.8) (end 155.1232 55.8) (width 0.2) (layer "F.Cu") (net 6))
 (segment (start 160 53.3647) (end 160 52.5805) (width 0.2) (layer "F.Cu") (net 6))
 (segment (start 157.2411 57.9192) (end 157.2411 60.5) (width 0.2) (layer "F.Cu") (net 20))
 (segment (start 157.2411 60.5) (end 156.5 60.5) (width 0.2) (layer "F.Cu") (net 20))
 (segment (start 162.1 58.75) (end 159.5725 61.2775) (width 0.2) (layer "F.Cu") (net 20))
 (segment (start 157.2411 60.7768) (end 157.2411 60.5) (width 0.2) (layer "F.Cu") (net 20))
 (segment (start 156.375 57.3) (end 156.6219 57.3) (width 0.2) (layer "F.Cu") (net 20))
 (segment (start 156.6219 57.3) (end 157.2411 57.9192) (width 0.2) (layer "F.Cu") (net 20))
 (segment (start 159.5725 61.2775) (end 157.7418 61.2775) (width 0.2) (layer "F.Cu") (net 20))
 (segment (start 157.7418 61.2775) (end 157.2411 60.7768) (width 0.2) (layer "F.Cu") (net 20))
 (segment (start 159.3273 58.3) (end 159.075 58.3) (width 0.2) (layer "F.Cu") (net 13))
 (segment (start 159.9848 56.7348) (end 159.9848 57.6425) (width 0.2) (layer "F.Cu") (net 13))
 (segment (start 159.9848 57.6425) (end 159.3273 58.3) (width 0.2) (layer "F.Cu") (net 13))
 (segment (start 158.55 55.3) (end 159.9848 56.7348) (width 0.2) (layer "F.Cu") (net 13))
 (segment (start 157.7092 54.4908) (end 159.5835 54.4908) (width 0.2) (layer "F.Cu") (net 12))
 (segment (start 156.9 55.3) (end 157.7092 54.4908) (width 0.2) (layer "F.Cu") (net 12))
 (segment (start 156.375 58.3) (end 156.1544 58.3) (width 0.2) (layer "F.Cu") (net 12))
 (segment (start 156.1544 58.3) (end 155.5007 57.6463) (width 0.2) (layer "F.Cu") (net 12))
 (segment (start 155.5007 57.6463) (end 155.5007 56.6993) (width 0.2) (layer "F.Cu") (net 12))
 (segment (start 161.9427 56.85) (end 162.1 56.85) (width 0.2) (layer "F.Cu") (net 12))
 (segment (start 155.5007 56.6993) (end 156.9 55.3) (width 0.2) (layer "F.Cu") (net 12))
 (segment (start 159.5835 54.4908) (end 161.9427 56.85) (width 0.2) (layer "F.Cu") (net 12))
 (segment (start 158.15 57.9837) (end 158.15 60.5) (width 0.2) (layer "F.Cu") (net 21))
 (segment (start 159.075 57.3) (end 158.8337 57.3) (width 0.2) (layer "F.Cu") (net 21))
 (segment (start 158.8337 57.3) (end 158.15 57.9837) (width 0.2) (layer "F.Cu") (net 21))
 (segment (start 139.05 51.85) (end 137.9 50.7) (width 0.2) (layer "F.Cu") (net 19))
 (segment (start 139.05 52.3) (end 139.05 51.85) (width 0.2) (layer "F.Cu") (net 19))
 (segment (start 138.3431 57) (end 137.4582 56.1151) (width 0.2) (layer "F.Cu") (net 1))
 (segment (start 135.4391 52.6115) (end 135.4391 49.5109) (width 0.2) (layer "F.Cu") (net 1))
 (segment (start 136.35 53.3) (end 136.1276 53.3) (width 0.2) (layer "F.Cu") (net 1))
 (segment (start 136.6655 53.3) (end 136.35 53.3) (width 0.2) (layer "F.Cu") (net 1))
 (segment (start 136.1276 53.3) (end 135.4391 52.6115) (width 0.2) (layer "F.Cu") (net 1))
 (segment (start 138.7 57) (end 138.3431 57) (width 0.2) (layer "F.Cu") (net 1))
 (segment (start 137.4582 54.0927) (end 136.6655 53.3) (width 0.2) (layer "F.Cu") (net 1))
 (segment (start 137.4582 56.1151) (end 137.4582 54.0927) (width 0.2) (layer "F.Cu") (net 1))
 (segment (start 135.4391 49.5109) (end 136.25 48.7) (width 0.2) (layer "F.Cu") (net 1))
 (segment (start 138.7 54.4291) (end 136.5709 52.3) (width 0.2) (layer "F.Cu") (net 3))
 (segment (start 136.35 52.3) (end 136.35 50.8) (width 0.2) (layer "F.Cu") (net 3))
 (segment (start 136.5709 52.3) (end 136.35 52.3) (width 0.2) (layer "F.Cu") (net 3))
 (segment (start 136.35 50.8) (end 136.25 50.7) (width 0.2) (layer "F.Cu") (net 3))
 (segment (start 138.7 55.1) (end 138.7 54.4291) (width 0.2) (layer "F.Cu") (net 3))
 (segment (start 139.05 53.3) (end 138.7997 53.3) (width 0.2) (layer "F.Cu") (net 18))
 (segment (start 137.1781 49.4219) (end 137.9 48.7) (width 0.2) (layer "F.Cu") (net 18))
 (segment (start 138.7997 53.3) (end 137.1781 51.6784) (width 0.2) (layer "F.Cu") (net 18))
 (segment (start 137.1781 51.6784) (end 137.1781 49.4219) (width 0.2) (layer "F.Cu") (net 18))
 (segment (start 157.125 52.9) (end 159.075 52.9) (width 0.2) (layer "F.Cu") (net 22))
 (segment (start 159.075 52.9) (end 159.175 53) (width 0.2) (layer "F.Cu") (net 22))
 (segment (start 140.325 58.8) (end 138.225 58.8) (width 0.2) (layer "F.Cu") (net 9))
 (segment (start 141.7 57.425) (end 140.325 58.8) (width 0.2) (layer "F.Cu") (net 9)))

